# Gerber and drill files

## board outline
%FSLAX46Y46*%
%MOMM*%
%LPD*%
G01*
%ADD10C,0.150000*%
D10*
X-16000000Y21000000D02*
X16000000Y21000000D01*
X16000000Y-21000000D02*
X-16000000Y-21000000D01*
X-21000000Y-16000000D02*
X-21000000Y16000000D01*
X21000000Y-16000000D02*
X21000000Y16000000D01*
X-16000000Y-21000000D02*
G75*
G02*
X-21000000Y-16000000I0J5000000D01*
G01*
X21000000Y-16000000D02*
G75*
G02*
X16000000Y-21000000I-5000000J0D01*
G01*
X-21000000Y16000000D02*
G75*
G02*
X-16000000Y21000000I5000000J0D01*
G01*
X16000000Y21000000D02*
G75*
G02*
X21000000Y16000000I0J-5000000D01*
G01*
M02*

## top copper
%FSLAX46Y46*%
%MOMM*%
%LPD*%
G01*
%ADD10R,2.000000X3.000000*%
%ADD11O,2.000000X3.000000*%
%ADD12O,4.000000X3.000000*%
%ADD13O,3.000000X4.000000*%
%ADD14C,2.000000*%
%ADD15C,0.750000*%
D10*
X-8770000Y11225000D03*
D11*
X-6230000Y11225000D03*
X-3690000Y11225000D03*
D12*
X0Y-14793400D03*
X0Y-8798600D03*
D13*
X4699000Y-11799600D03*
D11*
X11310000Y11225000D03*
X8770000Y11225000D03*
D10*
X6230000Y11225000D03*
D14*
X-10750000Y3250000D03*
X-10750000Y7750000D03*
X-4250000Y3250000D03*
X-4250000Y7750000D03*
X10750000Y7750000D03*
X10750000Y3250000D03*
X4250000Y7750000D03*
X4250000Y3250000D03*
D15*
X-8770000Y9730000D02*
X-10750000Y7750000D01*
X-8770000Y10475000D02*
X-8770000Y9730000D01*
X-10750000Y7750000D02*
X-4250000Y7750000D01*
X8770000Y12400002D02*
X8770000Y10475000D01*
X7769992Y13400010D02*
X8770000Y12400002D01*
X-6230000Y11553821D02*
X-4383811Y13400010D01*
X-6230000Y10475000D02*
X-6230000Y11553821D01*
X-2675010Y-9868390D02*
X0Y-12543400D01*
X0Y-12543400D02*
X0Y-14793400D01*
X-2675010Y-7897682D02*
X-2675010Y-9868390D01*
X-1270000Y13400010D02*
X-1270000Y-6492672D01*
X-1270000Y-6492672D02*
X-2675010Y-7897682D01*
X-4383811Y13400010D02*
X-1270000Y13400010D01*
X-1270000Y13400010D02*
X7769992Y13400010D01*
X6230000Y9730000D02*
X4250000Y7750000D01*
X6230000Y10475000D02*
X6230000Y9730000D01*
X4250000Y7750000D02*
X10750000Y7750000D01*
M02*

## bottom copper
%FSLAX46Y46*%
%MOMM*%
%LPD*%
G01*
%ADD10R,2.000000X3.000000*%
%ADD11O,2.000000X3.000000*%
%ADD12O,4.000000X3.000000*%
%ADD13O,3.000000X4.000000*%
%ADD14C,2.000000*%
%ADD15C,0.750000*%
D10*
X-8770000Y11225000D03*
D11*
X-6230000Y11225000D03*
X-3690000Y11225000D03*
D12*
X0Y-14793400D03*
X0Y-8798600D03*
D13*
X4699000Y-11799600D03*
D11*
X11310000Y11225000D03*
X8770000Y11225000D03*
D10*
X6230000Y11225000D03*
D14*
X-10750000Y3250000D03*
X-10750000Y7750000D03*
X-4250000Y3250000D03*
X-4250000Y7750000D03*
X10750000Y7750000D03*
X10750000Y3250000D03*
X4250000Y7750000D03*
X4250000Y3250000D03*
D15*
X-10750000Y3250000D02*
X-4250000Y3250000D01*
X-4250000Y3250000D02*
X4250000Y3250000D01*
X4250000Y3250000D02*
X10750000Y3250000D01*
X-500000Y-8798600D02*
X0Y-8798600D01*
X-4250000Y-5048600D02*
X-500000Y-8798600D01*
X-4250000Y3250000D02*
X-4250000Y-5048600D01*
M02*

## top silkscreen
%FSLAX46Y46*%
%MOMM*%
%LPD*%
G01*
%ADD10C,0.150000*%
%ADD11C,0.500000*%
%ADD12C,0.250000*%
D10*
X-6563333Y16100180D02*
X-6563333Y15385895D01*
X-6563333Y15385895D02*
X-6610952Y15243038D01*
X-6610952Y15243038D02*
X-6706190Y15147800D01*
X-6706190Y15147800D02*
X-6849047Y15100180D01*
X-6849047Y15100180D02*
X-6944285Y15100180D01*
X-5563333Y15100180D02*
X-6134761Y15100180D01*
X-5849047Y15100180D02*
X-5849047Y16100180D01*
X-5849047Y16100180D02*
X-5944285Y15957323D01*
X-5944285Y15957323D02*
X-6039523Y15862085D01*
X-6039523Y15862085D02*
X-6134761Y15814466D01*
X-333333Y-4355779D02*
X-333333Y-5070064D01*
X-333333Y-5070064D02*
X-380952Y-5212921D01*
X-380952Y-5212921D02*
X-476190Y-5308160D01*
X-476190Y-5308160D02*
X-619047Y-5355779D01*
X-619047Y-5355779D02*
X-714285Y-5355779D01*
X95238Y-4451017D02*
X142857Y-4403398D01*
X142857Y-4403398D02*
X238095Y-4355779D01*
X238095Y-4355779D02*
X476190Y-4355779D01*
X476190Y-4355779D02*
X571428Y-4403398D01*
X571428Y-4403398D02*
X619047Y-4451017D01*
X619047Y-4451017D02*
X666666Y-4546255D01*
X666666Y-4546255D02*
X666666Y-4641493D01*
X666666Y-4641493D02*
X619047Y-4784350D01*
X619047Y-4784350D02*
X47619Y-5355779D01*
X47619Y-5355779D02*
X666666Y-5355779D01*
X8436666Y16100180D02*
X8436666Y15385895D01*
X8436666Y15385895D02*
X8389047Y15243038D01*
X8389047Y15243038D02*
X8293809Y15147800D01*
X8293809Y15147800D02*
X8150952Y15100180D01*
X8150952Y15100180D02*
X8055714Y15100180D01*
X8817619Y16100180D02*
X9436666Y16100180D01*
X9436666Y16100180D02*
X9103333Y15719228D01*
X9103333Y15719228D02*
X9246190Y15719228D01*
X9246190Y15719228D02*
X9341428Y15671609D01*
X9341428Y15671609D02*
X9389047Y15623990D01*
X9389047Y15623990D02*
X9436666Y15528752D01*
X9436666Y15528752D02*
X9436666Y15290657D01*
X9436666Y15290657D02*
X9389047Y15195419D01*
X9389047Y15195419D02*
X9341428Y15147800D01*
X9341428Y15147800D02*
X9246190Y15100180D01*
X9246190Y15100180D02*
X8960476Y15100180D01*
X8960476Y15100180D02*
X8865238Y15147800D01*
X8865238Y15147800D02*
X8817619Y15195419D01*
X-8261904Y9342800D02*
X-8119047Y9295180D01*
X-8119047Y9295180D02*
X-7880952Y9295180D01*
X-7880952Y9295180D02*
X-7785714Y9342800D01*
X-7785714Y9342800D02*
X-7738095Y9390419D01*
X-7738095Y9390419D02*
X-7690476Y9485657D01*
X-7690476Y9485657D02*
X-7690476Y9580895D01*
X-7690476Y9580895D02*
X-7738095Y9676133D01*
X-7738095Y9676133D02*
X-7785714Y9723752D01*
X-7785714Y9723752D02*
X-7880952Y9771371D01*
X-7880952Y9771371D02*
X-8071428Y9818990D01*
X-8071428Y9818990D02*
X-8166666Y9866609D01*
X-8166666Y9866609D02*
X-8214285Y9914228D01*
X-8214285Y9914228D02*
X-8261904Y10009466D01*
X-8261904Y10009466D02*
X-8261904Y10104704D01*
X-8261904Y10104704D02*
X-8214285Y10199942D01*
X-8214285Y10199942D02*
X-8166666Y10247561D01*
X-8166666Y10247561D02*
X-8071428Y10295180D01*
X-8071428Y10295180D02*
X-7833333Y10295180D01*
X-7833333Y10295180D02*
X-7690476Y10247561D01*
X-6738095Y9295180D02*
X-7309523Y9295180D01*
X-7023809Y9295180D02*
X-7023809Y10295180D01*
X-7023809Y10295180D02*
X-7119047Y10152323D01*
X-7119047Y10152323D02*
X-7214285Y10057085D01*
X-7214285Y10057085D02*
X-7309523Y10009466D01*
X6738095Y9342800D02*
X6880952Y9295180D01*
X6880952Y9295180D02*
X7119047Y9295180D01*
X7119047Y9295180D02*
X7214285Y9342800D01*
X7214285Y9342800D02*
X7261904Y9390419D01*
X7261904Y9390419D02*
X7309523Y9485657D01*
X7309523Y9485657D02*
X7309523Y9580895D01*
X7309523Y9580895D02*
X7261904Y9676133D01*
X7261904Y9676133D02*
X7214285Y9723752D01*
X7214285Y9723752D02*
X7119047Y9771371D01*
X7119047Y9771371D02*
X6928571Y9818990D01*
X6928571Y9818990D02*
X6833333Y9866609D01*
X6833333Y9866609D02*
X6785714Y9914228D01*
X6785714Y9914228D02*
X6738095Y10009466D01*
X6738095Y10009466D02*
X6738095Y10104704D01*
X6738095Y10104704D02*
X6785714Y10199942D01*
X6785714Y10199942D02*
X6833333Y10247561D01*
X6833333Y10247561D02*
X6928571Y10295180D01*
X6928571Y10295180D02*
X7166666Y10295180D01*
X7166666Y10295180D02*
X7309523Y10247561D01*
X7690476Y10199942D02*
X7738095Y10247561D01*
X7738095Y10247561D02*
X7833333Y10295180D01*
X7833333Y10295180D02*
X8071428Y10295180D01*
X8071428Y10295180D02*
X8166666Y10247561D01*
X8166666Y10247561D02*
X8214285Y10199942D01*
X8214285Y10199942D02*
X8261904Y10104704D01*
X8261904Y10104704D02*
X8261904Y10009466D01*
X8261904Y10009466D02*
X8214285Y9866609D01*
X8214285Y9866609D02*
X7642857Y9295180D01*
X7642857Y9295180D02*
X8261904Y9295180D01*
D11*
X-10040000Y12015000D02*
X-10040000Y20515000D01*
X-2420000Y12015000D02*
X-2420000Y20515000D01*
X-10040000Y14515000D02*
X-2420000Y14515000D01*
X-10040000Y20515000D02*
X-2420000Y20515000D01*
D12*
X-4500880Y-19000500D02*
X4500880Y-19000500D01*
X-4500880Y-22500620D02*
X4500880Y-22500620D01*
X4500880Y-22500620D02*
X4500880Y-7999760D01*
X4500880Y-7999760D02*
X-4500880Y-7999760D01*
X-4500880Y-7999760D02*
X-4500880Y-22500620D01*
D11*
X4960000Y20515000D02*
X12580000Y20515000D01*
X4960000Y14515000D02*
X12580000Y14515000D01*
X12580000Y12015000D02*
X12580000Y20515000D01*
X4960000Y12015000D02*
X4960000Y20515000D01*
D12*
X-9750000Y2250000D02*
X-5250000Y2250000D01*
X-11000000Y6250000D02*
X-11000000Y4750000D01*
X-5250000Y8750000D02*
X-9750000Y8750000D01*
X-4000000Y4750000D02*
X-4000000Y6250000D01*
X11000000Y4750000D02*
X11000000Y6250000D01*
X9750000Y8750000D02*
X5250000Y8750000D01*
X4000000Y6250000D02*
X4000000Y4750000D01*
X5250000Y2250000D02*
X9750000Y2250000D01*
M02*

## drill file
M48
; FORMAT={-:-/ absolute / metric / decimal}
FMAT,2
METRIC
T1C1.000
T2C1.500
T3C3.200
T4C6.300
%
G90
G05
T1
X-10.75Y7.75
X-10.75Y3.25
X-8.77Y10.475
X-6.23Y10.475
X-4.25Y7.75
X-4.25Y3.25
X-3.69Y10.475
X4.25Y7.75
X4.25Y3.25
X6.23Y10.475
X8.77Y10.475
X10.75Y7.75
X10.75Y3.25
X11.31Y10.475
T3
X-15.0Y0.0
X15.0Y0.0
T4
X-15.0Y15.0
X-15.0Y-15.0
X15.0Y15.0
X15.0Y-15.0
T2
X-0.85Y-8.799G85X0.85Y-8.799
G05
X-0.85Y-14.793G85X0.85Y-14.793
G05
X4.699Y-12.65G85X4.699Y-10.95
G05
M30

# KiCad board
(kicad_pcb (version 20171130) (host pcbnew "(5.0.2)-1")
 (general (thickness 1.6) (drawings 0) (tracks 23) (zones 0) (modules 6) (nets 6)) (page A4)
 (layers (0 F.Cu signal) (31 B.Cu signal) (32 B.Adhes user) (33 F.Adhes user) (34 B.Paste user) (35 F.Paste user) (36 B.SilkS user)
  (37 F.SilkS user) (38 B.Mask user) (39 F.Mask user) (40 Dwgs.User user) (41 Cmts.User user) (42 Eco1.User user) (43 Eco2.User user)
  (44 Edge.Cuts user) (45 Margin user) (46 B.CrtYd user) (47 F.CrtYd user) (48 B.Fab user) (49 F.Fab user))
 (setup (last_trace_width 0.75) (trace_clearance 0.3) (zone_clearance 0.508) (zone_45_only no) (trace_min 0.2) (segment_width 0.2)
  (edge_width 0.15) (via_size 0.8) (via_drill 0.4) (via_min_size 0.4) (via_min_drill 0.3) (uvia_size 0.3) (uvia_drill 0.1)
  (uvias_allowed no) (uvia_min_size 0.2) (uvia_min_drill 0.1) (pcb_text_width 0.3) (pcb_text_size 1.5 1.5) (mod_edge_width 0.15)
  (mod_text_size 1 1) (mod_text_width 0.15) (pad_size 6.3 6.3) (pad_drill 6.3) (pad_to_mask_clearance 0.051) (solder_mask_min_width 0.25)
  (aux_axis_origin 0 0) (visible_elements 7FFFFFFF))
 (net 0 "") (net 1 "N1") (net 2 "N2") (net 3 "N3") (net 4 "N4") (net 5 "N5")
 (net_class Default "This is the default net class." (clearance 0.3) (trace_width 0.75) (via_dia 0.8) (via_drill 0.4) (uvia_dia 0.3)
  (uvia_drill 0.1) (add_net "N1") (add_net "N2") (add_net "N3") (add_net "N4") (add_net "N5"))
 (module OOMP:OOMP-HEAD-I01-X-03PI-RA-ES (layer F.Cu) (at -8.77 -10.935 90)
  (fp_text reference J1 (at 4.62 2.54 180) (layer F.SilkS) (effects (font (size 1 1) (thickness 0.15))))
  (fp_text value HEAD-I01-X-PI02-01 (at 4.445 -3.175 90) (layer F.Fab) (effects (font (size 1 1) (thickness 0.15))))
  (fp_line (start 1.08 -1.27) (end 9.58 -1.27) (layer F.SilkS) (width 0.5))
  (fp_line (start 1.08 6.35) (end 9.58 6.35) (layer F.SilkS) (width 0.5))
  (fp_line (start 3.58 -1.27) (end 3.58 6.35) (layer F.SilkS) (width 0.5))
  (fp_line (start 9.58 -1.27) (end 9.58 6.35) (layer F.SilkS) (width 0.5))
  (pad 1 thru_hole rect (at -0.46 0 90) (size 3 2) (drill 1 (offset 0.75 0)) (layers *.Cu *.Mask) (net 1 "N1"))
  (pad 2 thru_hole oval (at -0.46 2.54 90) (size 3 2) (drill 1 (offset 0.75 0)) (layers *.Cu *.Mask) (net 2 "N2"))
  (pad 3 thru_hole oval (at -0.46 5.08 90) (size 3 2) (drill 1 (offset 0.75 0)) (layers *.Cu *.Mask)))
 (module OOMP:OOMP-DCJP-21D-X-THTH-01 (layer F.Cu) (at 0 15 90)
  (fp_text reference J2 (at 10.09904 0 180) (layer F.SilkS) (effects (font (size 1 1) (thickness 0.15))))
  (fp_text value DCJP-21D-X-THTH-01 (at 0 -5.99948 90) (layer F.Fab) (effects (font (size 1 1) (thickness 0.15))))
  (fp_line (start -4.0005 -4.50088) (end -4.0005 4.50088) (layer F.SilkS) (width 0.25))
  (fp_line (start -7.50062 -4.50088) (end -7.50062 4.50088) (layer F.SilkS) (width 0.25))
  (fp_line (start -7.50062 4.50088) (end 7.00024 4.50088) (layer F.SilkS) (width 0.25))
  (fp_line (start 7.00024 4.50088) (end 7.00024 -4.50088) (layer F.SilkS) (width 0.25))
  (fp_line (start 7.00024 -4.50088) (end -7.50062 -4.50088) (layer F.SilkS) (width 0.25))
  (pad 2 thru_hole oval (at 0.2066 0 90) (size 3 4) (drill oval 1.5 3.2) (layers *.Cu *.Mask) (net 2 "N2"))
  (pad 1 thru_hole oval (at 6.2014 0 90) (size 3 4) (drill oval 1.5 3.2) (layers *.Cu *.Mask) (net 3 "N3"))
  (pad 3 thru_hole oval (at 3.2004 4.699 180) (size 3 4) (drill oval 1.5 3.2) (layers *.Cu *.Mask) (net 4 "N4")))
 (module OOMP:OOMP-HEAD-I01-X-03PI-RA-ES (layer F.Cu) (at 6.23 -10.935 90)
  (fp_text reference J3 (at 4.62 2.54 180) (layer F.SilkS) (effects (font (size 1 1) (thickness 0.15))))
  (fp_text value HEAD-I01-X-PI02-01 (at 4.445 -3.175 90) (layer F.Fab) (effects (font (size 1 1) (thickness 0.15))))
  (fp_line (start 9.58 -1.27) (end 9.58 6.35) (layer F.SilkS) (width 0.5))
  (fp_line (start 3.58 -1.27) (end 3.58 6.35) (layer F.SilkS) (width 0.5))
  (fp_line (start 1.08 6.35) (end 9.58 6.35) (layer F.SilkS) (width 0.5))
  (fp_line (start 1.08 -1.27) (end 9.58 -1.27) (layer F.SilkS) (width 0.5))
  (pad 3 thru_hole oval (at -0.46 5.08 90) (size 3 2) (drill 1 (offset 0.75 0)) (layers *.Cu *.Mask))
  (pad 2 thru_hole oval (at -0.46 2.54 90) (size 3 2) (drill 1 (offset 0.75 0)) (layers *.Cu *.Mask) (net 2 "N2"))
  (pad 1 thru_hole rect (at -0.46 0 90) (size 3 2) (drill 1 (offset 0.75 0)) (layers *.Cu *.Mask) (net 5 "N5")))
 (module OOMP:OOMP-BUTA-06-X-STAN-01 (layer F.Cu) (at -10.75 -7.75)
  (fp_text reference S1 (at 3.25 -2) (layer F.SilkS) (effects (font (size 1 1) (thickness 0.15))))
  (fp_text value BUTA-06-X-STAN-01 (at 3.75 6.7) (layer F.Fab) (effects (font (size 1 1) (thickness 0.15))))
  (fp_line (start 1 5.5) (end 5.5 5.5) (layer F.SilkS) (width 0.25))
  (fp_line (start -0.25 1.5) (end -0.25 3) (layer F.SilkS) (width 0.25))
  (fp_line (start 5.5 -1) (end 1 -1) (layer F.SilkS) (width 0.25))
  (fp_line (start 6.75 3) (end 6.75 1.5) (layer F.SilkS) (width 0.25))
  (pad 2 thru_hole circle (at 0 4.5 90) (size 2 2) (drill 1) (layers *.Cu *.Mask) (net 3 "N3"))
  (pad 1 thru_hole circle (at 0 0 90) (size 2 2) (drill 1) (layers *.Cu *.Mask) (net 1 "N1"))
  (pad 2 thru_hole circle (at 6.5 4.5 90) (size 2 2) (drill 1) (layers *.Cu *.Mask) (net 3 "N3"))
  (pad 1 thru_hole circle (at 6.5 0 90) (size 2 2) (drill 1) (layers *.Cu *.Mask) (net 1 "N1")))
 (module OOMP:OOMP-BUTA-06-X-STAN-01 (layer F.Cu) (at 4.25 -7.75)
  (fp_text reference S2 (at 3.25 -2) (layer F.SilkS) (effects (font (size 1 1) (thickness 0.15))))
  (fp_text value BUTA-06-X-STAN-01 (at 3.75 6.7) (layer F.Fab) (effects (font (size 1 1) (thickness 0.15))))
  (fp_line (start 6.75 3) (end 6.75 1.5) (layer F.SilkS) (width 0.25))
  (fp_line (start 5.5 -1) (end 1 -1) (layer F.SilkS) (width 0.25))
  (fp_line (start -0.25 1.5) (end -0.25 3) (layer F.SilkS) (width 0.25))
  (fp_line (start 1 5.5) (end 5.5 5.5) (layer F.SilkS) (width 0.25))
  (pad 1 thru_hole circle (at 6.5 0 90) (size 2 2) (drill 1) (layers *.Cu *.Mask) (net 5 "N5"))
  (pad 2 thru_hole circle (at 6.5 4.5 90) (size 2 2) (drill 1) (layers *.Cu *.Mask) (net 3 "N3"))
  (pad 1 thru_hole circle (at 0 0 90) (size 2 2) (drill 1) (layers *.Cu *.Mask) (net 5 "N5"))
  (pad 2 thru_hole circle (at 0 4.5 90) (size 2 2) (drill 1) (layers *.Cu *.Mask) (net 3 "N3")))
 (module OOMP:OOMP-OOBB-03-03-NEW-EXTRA (layer F.Cu) (at 0 0)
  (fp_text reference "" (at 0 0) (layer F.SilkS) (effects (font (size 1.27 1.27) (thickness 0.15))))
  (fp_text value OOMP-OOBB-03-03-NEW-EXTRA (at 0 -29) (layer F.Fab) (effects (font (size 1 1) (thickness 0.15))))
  (fp_line (start -16 -21) (end 16 -21) (layer Edge.Cuts) (width 0.15))
  (fp_line (start 16 21) (end -16 21) (layer Edge.Cuts) (width 0.15))
  (fp_line (start -21 16) (end -21 -16) (layer Edge.Cuts) (width 0.15))
  (fp_line (start 21 16) (end 21 -16) (layer Edge.Cuts) (width 0.15))
  (fp_arc (start -16 16) (end -16 21) (angle 90) (layer Edge.Cuts) (width 0.15))
  (fp_arc (start 16 16) (end 16 21) (angle -90) (layer Edge.Cuts) (width 0.15))
  (fp_arc (start -16 -16) (end -16 -21) (angle -90) (layer Edge.Cuts) (width 0.15))
  (fp_arc (start 16 -16) (end 16 -21) (angle 90) (layer Edge.Cuts) (width 0.15))
  (pad "" np_thru_hole circle (at 15 15) (size 6.3 6.3) (drill 6.3) (layers *.Cu *.Mask))
  (pad "" np_thru_hole circle (at 15 0) (size 3.2 3.2) (drill 3.2) (layers *.Cu *.Mask))
  (pad "" np_thru_hole circle (at 15 -15) (size 6.3 6.3) (drill 6.3) (layers *.Cu *.Mask))
  (pad "" np_thru_hole circle (at -15 15) (size 6.3 6.3) (drill 6.3) (layers *.Cu *.Mask))
  (pad "" np_thru_hole circle (at -15 0) (size 3.2 3.2) (drill 3.2) (layers *.Cu *.Mask))
  (pad "" np_thru_hole circle (at -15 -15) (size 6.3 6.3) (drill 6.3) (layers *.Cu *.Mask)))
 (segment (start -8.77 -9.73) (end -10.75 -7.75) (width 0.75) (layer F.Cu) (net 1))
 (segment (start -8.77 -10.475) (end -8.77 -9.73) (width 0.75) (layer F.Cu) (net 1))
 (segment (start -10.75 -7.75) (end -4.25 -7.75) (width 0.75) (layer F.Cu) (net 1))
 (segment (start 8.77 -12.400002) (end 8.77 -10.475) (width 0.75) (layer F.Cu) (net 2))
 (segment (start 7.769992 -13.40001) (end 8.77 -12.400002) (width 0.75) (layer F.Cu) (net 2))
 (segment (start -6.23 -11.553821) (end -4.383811 -13.40001) (width 0.75) (layer F.Cu) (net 2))
 (segment (start -6.23 -10.475) (end -6.23 -11.553821) (width 0.75) (layer F.Cu) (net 2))
 (segment (start -2.67501 9.86839) (end 0 12.5434) (width 0.75) (layer F.Cu) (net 2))
 (segment (start 0 12.5434) (end 0 14.7934) (width 0.75) (layer F.Cu) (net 2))
 (segment (start -2.67501 7.897682) (end -2.67501 9.86839) (width 0.75) (layer F.Cu) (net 2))
 (segment (start -1.27 -13.40001) (end -1.27 6.492672) (width 0.75) (layer F.Cu) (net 2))
 (segment (start -1.27 6.492672) (end -2.67501 7.897682) (width 0.75) (layer F.Cu) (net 2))
 (segment (start -4.383811 -13.40001) (end -1.27 -13.40001) (width 0.75) (layer F.Cu) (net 2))
 (segment (start -1.27 -13.40001) (end 7.769992 -13.40001) (width 0.75) (layer F.Cu) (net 2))
 (segment (start -10.75 -3.25) (end -4.25 -3.25) (width 0.75) (layer B.Cu) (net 3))
 (segment (start -4.25 -3.25) (end 4.25 -3.25) (width 0.75) (layer B.Cu) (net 3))
 (segment (start 4.25 -3.25) (end 10.75 -3.25) (width 0.75) (layer B.Cu) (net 3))
 (segment (start -0.5 8.7986) (end 0 8.7986) (width 0.75) (layer B.Cu) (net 3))
 (segment (start -4.25 5.0486) (end -0.5 8.7986) (width 0.75) (layer B.Cu) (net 3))
 (segment (start -4.25 -3.25) (end -4.25 5.0486) (width 0.75) (layer B.Cu) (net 3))
 (segment (start 6.23 -9.73) (end 4.25 -7.75) (width 0.75) (layer F.Cu) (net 5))
 (segment (start 6.23 -10.475) (end 6.23 -9.73) (width 0.75) (layer F.Cu) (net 5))
 (segment (start 4.25 -7.75) (end 10.75 -7.75) (width 0.75) (layer F.Cu) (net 5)))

